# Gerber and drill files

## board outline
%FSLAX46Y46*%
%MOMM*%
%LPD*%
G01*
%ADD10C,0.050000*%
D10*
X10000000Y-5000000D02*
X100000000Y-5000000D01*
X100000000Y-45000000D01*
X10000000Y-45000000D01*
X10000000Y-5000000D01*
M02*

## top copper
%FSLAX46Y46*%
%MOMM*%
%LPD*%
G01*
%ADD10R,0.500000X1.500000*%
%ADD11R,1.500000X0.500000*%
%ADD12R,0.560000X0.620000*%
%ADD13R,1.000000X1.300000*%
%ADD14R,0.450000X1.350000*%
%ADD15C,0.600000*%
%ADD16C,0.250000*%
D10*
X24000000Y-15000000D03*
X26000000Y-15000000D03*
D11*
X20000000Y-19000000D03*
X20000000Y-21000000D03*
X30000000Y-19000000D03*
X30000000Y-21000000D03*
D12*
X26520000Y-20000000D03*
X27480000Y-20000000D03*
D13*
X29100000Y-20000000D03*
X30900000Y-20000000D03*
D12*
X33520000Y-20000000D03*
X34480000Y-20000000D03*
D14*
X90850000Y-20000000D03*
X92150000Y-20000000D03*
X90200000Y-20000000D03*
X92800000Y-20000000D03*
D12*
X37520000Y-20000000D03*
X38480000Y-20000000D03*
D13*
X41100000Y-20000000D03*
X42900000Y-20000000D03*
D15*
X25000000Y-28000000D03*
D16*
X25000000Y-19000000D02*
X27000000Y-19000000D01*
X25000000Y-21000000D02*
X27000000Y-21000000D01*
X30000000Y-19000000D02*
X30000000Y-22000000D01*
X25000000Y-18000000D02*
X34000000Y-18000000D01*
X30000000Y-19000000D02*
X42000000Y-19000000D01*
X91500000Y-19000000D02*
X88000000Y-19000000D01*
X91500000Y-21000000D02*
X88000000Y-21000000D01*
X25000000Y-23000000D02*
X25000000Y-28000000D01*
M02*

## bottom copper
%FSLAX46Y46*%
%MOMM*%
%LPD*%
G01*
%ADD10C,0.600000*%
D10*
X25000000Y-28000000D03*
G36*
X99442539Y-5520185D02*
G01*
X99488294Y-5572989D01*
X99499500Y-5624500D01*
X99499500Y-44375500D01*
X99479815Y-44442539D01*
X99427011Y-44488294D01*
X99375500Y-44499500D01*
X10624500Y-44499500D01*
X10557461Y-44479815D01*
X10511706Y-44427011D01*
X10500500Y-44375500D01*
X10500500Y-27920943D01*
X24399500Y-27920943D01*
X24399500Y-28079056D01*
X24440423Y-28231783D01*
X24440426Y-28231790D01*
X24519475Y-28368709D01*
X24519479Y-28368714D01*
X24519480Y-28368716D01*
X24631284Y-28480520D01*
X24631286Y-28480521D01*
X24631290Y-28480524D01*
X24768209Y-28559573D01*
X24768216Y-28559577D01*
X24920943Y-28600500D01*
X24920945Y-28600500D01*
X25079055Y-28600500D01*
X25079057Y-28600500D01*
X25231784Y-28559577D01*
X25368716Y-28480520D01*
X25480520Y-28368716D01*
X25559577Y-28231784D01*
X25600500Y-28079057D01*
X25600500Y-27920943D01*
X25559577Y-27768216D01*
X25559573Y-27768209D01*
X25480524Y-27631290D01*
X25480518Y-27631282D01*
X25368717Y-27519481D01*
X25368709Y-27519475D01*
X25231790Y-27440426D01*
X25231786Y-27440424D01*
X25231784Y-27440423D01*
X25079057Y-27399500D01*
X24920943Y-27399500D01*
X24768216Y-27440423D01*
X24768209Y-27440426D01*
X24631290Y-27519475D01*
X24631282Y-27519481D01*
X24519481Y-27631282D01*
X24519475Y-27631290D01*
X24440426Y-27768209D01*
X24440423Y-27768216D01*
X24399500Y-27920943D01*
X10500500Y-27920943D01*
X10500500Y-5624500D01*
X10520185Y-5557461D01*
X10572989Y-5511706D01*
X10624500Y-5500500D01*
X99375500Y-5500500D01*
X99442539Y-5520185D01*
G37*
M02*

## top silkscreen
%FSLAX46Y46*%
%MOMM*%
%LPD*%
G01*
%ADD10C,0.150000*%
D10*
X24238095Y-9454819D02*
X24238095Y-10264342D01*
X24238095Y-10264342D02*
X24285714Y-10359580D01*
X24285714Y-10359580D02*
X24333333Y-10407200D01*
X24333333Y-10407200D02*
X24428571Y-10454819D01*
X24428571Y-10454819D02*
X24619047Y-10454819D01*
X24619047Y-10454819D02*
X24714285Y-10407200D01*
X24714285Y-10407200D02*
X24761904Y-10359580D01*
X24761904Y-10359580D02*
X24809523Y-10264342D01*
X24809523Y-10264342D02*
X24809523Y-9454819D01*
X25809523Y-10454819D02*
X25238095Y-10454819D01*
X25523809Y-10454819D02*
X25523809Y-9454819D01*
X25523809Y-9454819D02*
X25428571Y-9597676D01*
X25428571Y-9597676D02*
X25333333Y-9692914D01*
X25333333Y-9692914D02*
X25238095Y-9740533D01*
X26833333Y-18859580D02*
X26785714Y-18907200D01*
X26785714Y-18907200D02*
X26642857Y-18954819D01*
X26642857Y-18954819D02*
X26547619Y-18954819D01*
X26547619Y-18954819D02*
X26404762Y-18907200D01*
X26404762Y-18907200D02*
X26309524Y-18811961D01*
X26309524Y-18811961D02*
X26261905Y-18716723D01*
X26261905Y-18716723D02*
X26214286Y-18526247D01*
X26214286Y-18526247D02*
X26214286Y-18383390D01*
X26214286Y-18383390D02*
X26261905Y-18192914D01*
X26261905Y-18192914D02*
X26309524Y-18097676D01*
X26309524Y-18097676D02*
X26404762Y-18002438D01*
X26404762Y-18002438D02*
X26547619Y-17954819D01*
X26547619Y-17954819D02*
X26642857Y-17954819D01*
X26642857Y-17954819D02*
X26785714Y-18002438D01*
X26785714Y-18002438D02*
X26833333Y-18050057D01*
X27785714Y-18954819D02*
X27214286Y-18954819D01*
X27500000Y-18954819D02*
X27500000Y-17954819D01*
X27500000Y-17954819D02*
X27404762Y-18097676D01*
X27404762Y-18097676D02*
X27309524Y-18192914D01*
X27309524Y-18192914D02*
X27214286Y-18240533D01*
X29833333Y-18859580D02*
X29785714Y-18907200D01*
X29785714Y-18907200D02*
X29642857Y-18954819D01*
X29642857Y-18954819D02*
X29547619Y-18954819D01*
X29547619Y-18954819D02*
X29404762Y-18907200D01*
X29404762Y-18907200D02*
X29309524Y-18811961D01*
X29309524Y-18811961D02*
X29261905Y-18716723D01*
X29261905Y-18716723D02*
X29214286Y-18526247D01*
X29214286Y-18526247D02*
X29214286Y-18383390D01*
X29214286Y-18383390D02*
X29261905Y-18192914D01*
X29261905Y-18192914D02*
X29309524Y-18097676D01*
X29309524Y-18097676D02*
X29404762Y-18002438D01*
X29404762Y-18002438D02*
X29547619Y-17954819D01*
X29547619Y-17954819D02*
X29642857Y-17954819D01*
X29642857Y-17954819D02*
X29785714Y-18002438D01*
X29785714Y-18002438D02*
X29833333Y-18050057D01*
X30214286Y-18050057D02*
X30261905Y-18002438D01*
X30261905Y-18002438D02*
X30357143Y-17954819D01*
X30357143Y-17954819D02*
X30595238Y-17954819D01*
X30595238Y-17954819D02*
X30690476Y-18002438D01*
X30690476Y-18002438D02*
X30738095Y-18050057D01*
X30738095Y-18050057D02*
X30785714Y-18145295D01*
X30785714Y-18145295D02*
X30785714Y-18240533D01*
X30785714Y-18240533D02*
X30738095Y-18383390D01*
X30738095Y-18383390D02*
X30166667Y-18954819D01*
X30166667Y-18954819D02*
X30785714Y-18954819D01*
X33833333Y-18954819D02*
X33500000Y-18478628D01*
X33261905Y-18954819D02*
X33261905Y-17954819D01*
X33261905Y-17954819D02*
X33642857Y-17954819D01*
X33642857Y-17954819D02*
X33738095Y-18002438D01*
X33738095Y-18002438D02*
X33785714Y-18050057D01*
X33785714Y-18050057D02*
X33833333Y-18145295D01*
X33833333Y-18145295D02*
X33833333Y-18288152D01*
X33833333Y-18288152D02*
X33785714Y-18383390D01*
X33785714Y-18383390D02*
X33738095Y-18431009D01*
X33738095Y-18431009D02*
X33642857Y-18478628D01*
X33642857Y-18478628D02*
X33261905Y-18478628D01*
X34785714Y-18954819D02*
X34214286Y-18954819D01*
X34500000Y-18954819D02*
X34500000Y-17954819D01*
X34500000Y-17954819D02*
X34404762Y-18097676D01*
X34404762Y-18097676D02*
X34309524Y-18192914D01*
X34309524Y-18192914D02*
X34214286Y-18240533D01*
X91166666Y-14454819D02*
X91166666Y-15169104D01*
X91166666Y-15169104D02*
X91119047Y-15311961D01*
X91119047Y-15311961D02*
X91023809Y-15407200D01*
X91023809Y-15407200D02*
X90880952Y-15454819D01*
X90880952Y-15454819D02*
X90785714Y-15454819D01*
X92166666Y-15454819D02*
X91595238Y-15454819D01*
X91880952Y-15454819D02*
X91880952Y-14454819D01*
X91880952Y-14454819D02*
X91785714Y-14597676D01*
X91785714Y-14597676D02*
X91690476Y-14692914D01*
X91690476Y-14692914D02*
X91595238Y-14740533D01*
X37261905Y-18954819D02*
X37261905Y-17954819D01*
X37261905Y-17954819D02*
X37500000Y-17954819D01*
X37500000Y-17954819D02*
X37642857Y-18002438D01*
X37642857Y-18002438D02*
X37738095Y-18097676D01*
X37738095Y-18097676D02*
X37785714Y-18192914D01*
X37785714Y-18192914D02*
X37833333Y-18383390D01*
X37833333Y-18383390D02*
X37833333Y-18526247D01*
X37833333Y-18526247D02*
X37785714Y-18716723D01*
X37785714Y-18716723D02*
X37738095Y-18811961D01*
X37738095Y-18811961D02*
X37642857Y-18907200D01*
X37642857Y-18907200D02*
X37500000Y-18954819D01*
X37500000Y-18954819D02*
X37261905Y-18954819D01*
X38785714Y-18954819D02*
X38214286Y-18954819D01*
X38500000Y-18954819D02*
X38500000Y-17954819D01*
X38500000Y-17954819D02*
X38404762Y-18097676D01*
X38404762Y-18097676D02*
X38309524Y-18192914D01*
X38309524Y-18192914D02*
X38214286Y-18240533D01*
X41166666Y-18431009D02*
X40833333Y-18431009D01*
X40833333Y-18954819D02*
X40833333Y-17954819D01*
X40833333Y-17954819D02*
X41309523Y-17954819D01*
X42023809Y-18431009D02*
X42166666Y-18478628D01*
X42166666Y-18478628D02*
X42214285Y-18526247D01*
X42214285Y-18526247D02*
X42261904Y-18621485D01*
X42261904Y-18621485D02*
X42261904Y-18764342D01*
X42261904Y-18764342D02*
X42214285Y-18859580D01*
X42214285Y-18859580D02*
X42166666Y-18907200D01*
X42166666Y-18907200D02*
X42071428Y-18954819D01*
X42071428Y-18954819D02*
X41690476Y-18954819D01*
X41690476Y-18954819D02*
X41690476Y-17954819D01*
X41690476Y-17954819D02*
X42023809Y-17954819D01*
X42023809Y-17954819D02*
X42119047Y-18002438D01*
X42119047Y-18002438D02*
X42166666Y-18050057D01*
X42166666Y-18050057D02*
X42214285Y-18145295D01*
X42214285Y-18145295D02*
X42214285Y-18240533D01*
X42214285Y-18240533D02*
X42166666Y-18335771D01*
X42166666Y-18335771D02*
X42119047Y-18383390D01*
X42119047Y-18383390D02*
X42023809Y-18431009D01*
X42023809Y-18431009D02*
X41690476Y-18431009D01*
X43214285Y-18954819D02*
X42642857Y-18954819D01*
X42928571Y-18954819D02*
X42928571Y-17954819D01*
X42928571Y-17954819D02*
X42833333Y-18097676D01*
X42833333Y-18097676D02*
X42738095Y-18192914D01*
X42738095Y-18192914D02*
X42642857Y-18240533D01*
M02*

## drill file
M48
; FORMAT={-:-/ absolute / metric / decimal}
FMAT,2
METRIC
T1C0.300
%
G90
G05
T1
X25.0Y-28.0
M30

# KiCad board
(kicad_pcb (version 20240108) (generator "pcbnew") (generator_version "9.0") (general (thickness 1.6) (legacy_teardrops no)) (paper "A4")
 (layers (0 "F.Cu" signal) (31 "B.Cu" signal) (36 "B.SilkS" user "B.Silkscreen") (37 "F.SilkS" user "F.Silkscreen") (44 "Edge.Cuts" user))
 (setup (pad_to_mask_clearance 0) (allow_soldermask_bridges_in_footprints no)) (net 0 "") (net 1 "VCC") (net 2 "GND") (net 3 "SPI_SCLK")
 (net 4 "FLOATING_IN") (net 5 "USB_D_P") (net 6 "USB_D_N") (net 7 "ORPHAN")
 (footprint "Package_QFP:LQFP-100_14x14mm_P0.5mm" (at 25 20) (layer "F.Cu")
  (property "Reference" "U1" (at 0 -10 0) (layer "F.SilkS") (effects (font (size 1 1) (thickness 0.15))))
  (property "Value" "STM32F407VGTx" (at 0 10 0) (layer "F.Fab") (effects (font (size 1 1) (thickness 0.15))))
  (pad "VCC" smd rect (at -1 -5) (size 0.5 1.5) (layers "F.Cu" "F.Paste" "F.Mask") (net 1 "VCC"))
  (pad "GND" smd rect (at 1 -5) (size 0.5 1.5) (layers "F.Cu" "F.Paste" "F.Mask") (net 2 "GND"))
  (pad "DATA_IN" smd rect (at -5 -1) (size 1.5 0.5) (layers "F.Cu" "F.Paste" "F.Mask") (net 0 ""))
  (pad "DATA_OUT" smd rect (at -5 1) (size 1.5 0.5) (layers "F.Cu" "F.Paste" "F.Mask") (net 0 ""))
  (pad "SCLK" smd rect (at 5 -1) (size 1.5 0.5) (layers "F.Cu" "F.Paste" "F.Mask") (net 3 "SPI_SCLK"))
  (pad "FLOATING_IN" smd rect (at 5 1) (size 1.5 0.5) (layers "F.Cu" "F.Paste" "F.Mask") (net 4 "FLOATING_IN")))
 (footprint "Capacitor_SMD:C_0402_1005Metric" (at 27 20) (layer "F.Cu")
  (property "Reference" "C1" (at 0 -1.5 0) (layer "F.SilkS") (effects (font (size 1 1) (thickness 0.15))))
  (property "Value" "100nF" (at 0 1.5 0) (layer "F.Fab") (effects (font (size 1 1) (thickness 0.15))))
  (pad "1" smd rect (at -0.48 0) (size 0.56 0.62) (layers "F.Cu" "F.Paste" "F.Mask") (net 1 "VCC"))
  (pad "2" smd rect (at 0.48 0) (size 0.56 0.62) (layers "F.Cu" "F.Paste" "F.Mask") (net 2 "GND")))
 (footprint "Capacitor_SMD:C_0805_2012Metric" (at 30 20) (layer "F.Cu")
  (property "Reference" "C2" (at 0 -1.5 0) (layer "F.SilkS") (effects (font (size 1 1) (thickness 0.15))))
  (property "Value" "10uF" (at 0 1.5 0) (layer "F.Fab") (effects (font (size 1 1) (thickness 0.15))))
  (pad "1" smd rect (at -0.9 0) (size 1.0 1.3) (layers "F.Cu" "F.Paste" "F.Mask") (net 1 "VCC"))
  (pad "2" smd rect (at 0.9 0) (size 1.0 1.3) (layers "F.Cu" "F.Paste" "F.Mask") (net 2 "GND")))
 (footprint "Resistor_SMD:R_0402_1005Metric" (at 34 20) (layer "F.Cu")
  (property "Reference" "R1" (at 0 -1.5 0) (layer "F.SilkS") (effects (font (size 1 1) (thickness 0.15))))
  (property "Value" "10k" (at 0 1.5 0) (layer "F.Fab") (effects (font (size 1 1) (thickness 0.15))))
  (pad "1" smd rect (at -0.48 0) (size 0.56 0.62) (layers "F.Cu" "F.Paste" "F.Mask") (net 1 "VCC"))
  (pad "2" smd rect (at 0.48 0) (size 0.56 0.62) (layers "F.Cu" "F.Paste" "F.Mask") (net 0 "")))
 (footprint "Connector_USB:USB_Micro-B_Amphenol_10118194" (at 91.5 20) (layer "F.Cu")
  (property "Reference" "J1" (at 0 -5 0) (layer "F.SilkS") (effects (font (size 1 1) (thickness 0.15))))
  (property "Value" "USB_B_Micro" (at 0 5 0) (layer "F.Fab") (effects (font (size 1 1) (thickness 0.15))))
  (pad "D+" smd rect (at -0.65 0) (size 0.45 1.35) (layers "F.Cu" "F.Paste" "F.Mask") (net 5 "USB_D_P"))
  (pad "D-" smd rect (at 0.65 0) (size 0.45 1.35) (layers "F.Cu" "F.Paste" "F.Mask") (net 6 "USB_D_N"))
  (pad "VBUS" smd rect (at -1.3 0) (size 0.45 1.35) (layers "F.Cu" "F.Paste" "F.Mask") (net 1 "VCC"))
  (pad "GND" smd rect (at 1.3 0) (size 0.45 1.35) (layers "F.Cu" "F.Paste" "F.Mask") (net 2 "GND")))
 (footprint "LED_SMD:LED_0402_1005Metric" (at 38 20) (layer "F.Cu")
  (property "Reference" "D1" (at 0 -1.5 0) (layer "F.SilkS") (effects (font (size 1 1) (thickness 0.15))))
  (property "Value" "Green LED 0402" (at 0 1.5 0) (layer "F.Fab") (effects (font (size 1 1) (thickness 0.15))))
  (pad "A" smd rect (at -0.48 0) (size 0.56 0.62) (layers "F.Cu" "F.Paste" "F.Mask") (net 1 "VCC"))
  (pad "K" smd rect (at 0.48 0) (size 0.56 0.62) (layers "F.Cu" "F.Paste" "F.Mask") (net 2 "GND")))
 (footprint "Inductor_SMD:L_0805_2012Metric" (at 42 20) (layer "F.Cu")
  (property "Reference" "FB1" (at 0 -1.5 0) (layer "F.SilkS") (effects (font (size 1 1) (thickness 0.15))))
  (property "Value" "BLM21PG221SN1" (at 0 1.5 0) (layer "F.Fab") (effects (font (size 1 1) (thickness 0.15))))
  (pad "1" smd rect (at -0.9 0) (size 1.0 1.3) (layers "F.Cu" "F.Paste" "F.Mask") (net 1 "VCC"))
  (pad "2" smd rect (at 0.9 0) (size 1.0 1.3) (layers "F.Cu" "F.Paste" "F.Mask") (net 2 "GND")))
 (segment (start 25 19) (end 27 19) (width 0.25) (layer "F.Cu") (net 1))
 (segment (start 25 21) (end 27 21) (width 0.25) (layer "F.Cu") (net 2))
 (segment (start 30 19) (end 30 22) (width 0.25) (layer "F.Cu") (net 1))
 (segment (start 25 18) (end 34 18) (width 0.25) (layer "F.Cu") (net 1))
 (segment (start 30 19) (end 42 19) (width 0.25) (layer "F.Cu") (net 1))
 (segment (start 91.5 19) (end 88 19) (width 0.25) (layer "F.Cu") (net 5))
 (segment (start 91.5 21) (end 88 21) (width 0.25) (layer "F.Cu") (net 6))
 (segment (start 25 23) (end 25 28) (width 0.25) (layer "F.Cu") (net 3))
 (via (at 25 28) (size 0.6) (drill 0.3) (layers "F.Cu" "B.Cu") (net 3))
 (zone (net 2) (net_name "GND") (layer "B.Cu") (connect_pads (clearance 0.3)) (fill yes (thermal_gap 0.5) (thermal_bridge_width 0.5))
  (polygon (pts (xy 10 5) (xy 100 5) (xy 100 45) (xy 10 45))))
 (gr_rect (start 10 5) (end 100 45) (layer "Edge.Cuts") (width 0.05)))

